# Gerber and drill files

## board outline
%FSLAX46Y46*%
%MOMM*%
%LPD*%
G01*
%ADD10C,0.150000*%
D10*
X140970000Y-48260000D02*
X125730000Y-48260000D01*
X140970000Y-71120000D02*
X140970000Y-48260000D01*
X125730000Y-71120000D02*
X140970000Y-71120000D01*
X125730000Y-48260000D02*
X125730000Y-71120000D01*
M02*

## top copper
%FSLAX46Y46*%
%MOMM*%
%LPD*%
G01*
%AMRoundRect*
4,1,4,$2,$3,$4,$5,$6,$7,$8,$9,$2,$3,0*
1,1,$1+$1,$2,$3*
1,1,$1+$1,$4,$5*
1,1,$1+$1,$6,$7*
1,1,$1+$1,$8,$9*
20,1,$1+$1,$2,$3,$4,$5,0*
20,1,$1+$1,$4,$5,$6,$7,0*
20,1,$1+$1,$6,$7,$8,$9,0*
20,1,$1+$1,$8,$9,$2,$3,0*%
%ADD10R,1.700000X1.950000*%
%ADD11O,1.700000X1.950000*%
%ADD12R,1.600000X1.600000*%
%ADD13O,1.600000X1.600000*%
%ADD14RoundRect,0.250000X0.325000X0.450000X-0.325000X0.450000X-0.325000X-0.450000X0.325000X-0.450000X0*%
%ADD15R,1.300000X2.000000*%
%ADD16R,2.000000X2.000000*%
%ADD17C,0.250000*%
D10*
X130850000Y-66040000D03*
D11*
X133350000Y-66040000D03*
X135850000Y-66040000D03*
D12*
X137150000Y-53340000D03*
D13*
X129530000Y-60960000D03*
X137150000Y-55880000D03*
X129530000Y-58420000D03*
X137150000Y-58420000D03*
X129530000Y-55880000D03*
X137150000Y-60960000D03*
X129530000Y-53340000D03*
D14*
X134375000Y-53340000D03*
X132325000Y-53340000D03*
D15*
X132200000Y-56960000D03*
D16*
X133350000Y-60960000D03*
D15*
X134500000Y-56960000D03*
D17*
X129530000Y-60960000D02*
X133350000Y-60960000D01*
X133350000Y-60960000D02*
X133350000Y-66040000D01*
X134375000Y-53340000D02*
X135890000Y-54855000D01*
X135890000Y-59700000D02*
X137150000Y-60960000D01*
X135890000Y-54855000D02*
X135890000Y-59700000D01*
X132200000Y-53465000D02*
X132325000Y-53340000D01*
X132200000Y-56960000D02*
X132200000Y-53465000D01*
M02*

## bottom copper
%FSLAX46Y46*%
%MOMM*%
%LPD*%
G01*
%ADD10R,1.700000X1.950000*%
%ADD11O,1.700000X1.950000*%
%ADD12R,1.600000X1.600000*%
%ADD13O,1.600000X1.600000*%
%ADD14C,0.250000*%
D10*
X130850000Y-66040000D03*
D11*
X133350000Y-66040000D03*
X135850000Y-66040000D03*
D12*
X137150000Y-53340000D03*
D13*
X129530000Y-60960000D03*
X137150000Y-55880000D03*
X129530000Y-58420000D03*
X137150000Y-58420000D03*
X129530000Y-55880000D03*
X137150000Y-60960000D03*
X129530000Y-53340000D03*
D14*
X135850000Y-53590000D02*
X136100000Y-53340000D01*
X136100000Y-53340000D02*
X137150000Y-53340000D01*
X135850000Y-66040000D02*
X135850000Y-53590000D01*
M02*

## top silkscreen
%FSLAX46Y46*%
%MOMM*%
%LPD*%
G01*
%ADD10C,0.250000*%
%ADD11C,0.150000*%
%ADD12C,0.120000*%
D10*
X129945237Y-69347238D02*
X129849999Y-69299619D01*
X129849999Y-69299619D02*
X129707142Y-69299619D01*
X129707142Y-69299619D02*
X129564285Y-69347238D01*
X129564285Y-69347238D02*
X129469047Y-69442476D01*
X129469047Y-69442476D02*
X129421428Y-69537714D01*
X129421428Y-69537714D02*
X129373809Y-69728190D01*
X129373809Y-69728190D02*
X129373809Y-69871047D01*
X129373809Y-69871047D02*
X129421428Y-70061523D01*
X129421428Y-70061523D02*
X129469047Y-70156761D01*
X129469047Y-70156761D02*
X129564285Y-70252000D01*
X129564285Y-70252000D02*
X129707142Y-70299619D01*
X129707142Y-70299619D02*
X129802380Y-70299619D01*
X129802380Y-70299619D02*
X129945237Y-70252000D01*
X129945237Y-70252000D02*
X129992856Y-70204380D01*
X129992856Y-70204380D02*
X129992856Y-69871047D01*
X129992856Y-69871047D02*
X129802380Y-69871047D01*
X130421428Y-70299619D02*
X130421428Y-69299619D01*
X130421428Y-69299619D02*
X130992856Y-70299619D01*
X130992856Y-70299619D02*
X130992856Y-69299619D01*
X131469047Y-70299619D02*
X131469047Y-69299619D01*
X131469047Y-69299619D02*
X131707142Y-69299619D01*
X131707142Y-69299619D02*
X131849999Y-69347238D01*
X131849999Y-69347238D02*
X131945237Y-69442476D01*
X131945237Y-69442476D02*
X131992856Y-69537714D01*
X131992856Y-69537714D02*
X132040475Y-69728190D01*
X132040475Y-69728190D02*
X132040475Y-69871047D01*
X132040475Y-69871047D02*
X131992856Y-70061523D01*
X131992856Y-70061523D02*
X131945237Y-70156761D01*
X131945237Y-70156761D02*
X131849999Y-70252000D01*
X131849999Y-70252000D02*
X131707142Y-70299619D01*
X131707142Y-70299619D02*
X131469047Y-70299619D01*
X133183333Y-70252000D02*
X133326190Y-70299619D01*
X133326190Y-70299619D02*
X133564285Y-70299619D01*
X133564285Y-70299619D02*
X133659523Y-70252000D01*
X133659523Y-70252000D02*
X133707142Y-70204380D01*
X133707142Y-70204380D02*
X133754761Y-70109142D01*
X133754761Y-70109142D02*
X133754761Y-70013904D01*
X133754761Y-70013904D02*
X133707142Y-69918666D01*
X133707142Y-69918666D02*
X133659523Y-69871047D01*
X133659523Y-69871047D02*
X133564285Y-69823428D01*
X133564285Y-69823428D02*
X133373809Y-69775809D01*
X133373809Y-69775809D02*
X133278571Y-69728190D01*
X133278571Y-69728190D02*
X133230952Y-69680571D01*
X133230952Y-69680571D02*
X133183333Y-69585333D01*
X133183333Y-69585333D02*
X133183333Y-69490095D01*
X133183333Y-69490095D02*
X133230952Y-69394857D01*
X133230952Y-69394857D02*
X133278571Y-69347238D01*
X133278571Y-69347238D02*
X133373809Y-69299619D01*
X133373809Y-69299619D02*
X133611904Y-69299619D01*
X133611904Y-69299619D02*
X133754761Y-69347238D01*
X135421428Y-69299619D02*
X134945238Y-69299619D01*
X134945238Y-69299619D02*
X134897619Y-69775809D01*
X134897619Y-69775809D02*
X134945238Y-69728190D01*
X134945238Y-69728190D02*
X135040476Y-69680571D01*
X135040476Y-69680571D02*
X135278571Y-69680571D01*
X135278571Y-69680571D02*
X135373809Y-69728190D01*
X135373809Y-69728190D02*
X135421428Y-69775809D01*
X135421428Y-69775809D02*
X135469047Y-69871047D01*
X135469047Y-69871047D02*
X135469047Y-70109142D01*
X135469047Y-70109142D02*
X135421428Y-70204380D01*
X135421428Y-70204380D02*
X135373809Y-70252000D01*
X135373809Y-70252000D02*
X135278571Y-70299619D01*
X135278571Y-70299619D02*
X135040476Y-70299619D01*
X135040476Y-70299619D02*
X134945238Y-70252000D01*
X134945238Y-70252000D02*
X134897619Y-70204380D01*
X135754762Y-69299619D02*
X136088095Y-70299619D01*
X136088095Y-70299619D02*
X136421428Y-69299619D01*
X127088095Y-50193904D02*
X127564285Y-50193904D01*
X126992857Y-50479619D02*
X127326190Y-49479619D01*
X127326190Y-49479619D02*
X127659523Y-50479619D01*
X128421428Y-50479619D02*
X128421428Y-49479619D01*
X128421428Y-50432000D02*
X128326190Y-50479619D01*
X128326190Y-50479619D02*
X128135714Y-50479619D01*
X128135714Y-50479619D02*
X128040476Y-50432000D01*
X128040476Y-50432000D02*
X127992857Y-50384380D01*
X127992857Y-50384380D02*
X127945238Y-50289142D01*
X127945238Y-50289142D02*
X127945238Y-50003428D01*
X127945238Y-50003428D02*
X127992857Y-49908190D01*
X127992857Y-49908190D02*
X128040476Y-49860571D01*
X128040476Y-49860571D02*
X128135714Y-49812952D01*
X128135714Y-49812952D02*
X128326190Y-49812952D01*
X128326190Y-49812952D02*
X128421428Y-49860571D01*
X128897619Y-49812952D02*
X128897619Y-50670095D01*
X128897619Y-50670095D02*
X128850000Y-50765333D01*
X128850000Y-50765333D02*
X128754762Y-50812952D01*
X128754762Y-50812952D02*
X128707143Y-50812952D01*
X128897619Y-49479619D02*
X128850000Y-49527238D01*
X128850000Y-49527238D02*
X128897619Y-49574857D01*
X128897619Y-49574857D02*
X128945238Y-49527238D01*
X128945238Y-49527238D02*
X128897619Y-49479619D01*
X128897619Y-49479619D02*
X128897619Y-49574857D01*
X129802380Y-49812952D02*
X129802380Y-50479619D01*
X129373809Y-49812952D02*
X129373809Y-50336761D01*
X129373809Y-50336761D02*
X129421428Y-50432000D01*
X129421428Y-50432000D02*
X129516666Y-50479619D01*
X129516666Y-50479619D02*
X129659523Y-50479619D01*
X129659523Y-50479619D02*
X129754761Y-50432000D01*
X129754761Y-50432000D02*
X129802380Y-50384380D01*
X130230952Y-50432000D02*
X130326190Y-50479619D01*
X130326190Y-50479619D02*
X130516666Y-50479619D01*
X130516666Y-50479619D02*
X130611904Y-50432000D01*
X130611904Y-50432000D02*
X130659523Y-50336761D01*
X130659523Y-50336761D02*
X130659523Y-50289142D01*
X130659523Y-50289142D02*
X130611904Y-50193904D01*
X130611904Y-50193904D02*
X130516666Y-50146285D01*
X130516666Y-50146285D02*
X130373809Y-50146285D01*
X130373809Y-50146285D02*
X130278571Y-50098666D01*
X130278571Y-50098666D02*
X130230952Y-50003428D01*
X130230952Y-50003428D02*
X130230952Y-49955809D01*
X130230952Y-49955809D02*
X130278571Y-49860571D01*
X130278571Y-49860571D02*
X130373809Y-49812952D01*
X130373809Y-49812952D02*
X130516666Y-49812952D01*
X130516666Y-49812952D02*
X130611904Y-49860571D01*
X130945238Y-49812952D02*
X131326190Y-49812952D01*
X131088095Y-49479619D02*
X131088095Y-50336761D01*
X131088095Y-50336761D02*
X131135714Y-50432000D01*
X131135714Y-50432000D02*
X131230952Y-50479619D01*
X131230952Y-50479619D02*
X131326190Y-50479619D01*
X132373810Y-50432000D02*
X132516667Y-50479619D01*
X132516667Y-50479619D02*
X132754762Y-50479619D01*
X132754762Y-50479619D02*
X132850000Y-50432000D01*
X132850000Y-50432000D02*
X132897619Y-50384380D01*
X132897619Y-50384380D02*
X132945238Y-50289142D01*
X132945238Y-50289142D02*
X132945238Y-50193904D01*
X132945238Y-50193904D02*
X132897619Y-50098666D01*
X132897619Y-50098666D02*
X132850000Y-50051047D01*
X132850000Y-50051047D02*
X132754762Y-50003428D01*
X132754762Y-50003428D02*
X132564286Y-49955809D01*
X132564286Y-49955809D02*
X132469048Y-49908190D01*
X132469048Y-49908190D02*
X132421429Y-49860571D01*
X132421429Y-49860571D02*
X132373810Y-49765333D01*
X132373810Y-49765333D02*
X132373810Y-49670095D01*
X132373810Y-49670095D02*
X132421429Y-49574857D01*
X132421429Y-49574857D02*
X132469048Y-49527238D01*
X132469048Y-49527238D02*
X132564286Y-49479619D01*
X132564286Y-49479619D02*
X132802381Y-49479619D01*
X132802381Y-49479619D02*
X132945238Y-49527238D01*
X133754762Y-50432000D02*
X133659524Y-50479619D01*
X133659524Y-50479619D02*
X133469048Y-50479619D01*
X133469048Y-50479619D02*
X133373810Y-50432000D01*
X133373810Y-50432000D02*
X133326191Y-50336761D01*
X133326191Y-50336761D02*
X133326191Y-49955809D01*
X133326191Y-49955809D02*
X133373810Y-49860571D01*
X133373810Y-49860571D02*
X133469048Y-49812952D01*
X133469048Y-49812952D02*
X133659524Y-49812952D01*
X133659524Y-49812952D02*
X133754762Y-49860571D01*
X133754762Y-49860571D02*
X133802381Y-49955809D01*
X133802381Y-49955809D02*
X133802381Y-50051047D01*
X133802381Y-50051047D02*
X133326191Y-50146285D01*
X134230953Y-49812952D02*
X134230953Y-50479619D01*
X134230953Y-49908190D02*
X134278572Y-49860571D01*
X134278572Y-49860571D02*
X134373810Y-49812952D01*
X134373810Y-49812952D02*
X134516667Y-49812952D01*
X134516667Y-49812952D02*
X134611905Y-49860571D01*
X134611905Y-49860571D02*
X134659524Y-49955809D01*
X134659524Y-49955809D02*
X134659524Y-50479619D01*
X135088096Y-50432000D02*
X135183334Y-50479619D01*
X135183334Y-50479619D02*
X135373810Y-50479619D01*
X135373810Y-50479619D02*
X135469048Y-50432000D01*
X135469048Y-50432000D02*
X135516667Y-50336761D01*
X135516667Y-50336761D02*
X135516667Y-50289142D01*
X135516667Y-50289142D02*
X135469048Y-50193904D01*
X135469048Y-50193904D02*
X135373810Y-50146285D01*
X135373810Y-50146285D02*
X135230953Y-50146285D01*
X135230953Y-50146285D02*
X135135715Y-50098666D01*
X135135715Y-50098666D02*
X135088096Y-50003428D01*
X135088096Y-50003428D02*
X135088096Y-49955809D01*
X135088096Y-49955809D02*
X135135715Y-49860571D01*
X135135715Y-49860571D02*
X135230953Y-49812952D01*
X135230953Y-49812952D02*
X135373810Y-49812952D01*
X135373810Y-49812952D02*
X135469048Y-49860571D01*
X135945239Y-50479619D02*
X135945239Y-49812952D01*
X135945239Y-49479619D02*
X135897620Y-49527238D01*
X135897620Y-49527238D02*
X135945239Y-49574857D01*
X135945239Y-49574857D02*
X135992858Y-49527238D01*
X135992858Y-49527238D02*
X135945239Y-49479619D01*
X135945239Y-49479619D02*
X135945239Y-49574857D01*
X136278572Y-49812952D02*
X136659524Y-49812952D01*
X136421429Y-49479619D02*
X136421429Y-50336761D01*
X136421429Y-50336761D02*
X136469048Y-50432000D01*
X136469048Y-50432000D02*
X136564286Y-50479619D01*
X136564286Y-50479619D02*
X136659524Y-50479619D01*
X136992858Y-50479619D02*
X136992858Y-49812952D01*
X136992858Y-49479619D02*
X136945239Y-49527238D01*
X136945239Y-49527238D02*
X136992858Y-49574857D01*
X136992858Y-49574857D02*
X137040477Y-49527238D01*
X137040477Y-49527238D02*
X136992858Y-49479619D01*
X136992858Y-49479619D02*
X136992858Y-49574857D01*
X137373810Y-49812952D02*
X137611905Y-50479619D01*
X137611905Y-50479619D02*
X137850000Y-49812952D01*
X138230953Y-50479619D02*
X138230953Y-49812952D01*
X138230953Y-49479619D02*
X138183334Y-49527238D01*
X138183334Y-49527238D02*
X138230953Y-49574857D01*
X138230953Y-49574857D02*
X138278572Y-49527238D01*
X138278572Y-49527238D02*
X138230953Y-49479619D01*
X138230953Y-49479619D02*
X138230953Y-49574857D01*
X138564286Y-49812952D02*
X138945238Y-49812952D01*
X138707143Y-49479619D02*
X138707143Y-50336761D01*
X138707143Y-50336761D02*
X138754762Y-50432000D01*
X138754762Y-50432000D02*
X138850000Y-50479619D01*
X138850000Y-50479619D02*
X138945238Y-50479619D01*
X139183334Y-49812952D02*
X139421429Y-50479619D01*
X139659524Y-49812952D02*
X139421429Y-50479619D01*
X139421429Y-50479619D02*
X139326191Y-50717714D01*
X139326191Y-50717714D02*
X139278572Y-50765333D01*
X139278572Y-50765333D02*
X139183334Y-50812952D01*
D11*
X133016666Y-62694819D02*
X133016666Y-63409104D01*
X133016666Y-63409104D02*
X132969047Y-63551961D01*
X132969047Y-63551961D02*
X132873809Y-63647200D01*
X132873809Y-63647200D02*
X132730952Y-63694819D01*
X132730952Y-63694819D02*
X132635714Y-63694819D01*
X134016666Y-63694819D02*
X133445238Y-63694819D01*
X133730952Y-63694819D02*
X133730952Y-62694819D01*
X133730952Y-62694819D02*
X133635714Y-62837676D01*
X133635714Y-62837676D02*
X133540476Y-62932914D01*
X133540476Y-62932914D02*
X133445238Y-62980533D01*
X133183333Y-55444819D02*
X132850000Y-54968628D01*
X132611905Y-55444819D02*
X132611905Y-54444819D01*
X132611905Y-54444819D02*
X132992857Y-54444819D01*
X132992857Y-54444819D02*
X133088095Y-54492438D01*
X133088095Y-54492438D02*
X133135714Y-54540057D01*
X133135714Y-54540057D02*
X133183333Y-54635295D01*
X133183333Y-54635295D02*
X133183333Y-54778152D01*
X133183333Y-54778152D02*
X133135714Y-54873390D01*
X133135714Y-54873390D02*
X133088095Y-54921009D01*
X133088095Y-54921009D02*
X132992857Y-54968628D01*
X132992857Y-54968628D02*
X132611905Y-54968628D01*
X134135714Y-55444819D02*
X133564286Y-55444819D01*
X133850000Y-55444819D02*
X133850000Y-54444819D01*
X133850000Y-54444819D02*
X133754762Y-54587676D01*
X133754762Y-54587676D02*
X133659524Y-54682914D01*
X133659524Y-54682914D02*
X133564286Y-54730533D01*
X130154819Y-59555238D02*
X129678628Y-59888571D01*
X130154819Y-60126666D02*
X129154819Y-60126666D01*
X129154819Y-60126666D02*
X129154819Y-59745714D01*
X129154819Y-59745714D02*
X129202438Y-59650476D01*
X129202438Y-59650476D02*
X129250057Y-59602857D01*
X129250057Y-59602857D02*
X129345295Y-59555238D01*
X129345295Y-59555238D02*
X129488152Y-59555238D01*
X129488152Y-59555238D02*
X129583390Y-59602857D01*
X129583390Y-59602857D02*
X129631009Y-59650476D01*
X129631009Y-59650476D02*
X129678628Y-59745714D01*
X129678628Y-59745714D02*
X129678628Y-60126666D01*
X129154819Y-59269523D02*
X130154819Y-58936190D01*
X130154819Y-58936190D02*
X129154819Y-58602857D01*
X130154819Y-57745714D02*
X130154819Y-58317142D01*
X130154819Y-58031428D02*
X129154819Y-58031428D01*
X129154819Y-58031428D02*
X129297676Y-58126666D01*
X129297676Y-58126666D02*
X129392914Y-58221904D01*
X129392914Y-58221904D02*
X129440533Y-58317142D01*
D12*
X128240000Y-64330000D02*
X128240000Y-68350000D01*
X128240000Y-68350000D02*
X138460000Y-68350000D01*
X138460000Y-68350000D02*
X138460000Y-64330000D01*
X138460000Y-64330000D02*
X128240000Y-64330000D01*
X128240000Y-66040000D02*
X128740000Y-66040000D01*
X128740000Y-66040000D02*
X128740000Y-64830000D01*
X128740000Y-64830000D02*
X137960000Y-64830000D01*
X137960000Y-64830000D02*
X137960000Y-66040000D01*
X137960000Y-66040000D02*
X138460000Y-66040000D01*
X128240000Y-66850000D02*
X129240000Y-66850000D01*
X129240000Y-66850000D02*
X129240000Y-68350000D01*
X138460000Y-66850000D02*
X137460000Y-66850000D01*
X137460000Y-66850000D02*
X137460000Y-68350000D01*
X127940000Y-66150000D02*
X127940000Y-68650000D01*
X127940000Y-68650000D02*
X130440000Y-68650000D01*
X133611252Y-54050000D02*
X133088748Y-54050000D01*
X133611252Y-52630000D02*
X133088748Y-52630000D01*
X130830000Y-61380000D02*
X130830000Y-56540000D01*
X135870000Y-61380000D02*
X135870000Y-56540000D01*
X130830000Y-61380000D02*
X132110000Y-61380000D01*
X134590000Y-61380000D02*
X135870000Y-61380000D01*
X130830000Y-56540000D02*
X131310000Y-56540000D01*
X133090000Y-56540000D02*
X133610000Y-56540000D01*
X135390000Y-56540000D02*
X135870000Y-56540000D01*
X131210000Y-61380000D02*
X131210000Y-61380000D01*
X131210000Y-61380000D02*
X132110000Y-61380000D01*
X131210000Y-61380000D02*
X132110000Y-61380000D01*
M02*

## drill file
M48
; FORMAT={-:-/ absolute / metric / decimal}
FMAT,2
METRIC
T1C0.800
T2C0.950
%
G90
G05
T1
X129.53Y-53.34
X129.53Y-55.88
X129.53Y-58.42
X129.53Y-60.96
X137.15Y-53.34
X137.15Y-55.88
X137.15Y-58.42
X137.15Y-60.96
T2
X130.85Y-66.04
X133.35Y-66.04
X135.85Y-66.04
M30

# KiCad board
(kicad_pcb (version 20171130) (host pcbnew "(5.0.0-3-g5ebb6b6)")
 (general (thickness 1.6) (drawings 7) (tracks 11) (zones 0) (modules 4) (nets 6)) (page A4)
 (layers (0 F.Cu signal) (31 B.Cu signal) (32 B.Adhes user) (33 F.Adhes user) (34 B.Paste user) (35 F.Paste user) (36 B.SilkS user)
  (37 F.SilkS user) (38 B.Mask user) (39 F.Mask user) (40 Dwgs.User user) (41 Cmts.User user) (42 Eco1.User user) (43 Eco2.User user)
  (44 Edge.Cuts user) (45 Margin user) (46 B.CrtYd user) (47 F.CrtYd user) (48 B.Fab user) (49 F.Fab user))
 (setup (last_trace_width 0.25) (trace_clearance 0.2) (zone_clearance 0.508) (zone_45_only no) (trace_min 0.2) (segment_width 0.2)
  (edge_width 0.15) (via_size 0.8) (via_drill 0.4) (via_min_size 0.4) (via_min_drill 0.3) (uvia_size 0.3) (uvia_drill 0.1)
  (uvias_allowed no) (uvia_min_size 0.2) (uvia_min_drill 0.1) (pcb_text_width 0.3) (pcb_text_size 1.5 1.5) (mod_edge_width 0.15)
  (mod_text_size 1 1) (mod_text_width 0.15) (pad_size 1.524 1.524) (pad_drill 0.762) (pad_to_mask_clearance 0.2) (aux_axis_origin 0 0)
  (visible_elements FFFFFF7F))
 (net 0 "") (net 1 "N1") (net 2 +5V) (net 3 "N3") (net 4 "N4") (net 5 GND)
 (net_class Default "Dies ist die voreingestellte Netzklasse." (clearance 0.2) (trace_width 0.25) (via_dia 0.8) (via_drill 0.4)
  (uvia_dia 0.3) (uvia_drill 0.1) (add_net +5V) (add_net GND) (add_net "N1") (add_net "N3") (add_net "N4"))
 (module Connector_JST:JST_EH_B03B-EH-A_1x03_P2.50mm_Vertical (layer F.Cu) (at 130.85 66.04)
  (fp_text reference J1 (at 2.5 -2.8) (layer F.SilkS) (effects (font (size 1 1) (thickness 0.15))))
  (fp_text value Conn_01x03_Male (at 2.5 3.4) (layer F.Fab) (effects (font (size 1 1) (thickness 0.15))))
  (fp_line (start -2.61 -1.71) (end -2.61 2.31) (layer F.SilkS) (width 0.12))
  (fp_line (start -2.61 2.31) (end 7.61 2.31) (layer F.SilkS) (width 0.12))
  (fp_line (start 7.61 2.31) (end 7.61 -1.71) (layer F.SilkS) (width 0.12))
  (fp_line (start 7.61 -1.71) (end -2.61 -1.71) (layer F.SilkS) (width 0.12))
  (fp_line (start -2.61 0) (end -2.11 0) (layer F.SilkS) (width 0.12))
  (fp_line (start -2.11 0) (end -2.11 -1.21) (layer F.SilkS) (width 0.12))
  (fp_line (start -2.11 -1.21) (end 7.11 -1.21) (layer F.SilkS) (width 0.12))
  (fp_line (start 7.11 -1.21) (end 7.11 0) (layer F.SilkS) (width 0.12))
  (fp_line (start 7.11 0) (end 7.61 0) (layer F.SilkS) (width 0.12))
  (fp_line (start -2.61 0.81) (end -1.61 0.81) (layer F.SilkS) (width 0.12))
  (fp_line (start -1.61 0.81) (end -1.61 2.31) (layer F.SilkS) (width 0.12))
  (fp_line (start 7.61 0.81) (end 6.61 0.81) (layer F.SilkS) (width 0.12))
  (fp_line (start 6.61 0.81) (end 6.61 2.31) (layer F.SilkS) (width 0.12))
  (fp_line (start -2.91 0.11) (end -2.91 2.61) (layer F.SilkS) (width 0.12))
  (fp_line (start -2.91 2.61) (end -0.41 2.61) (layer F.SilkS) (width 0.12))
  (pad 1 thru_hole rect (at 0 0) (size 1.7 1.95) (drill 0.95) (layers *.Cu *.Mask))
  (pad 2 thru_hole oval (at 2.5 0) (size 1.7 1.95) (drill 0.95) (layers *.Cu *.Mask) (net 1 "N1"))
  (pad 3 thru_hole oval (at 5 0) (size 1.7 1.95) (drill 0.95) (layers *.Cu *.Mask) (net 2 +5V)))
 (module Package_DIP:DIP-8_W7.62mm (layer B.Cu) (at 137.15 53.34 180)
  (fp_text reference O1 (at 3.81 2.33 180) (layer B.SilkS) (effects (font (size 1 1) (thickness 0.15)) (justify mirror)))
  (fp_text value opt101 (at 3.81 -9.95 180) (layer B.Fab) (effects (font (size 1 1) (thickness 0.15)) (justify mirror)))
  (pad 1 thru_hole rect (at 0 0 180) (size 1.6 1.6) (drill 0.8) (layers *.Cu *.Mask) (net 2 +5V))
  (pad 5 thru_hole oval (at 7.62 -7.62 180) (size 1.6 1.6) (drill 0.8) (layers *.Cu *.Mask) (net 1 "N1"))
  (pad 2 thru_hole oval (at 0 -2.54 180) (size 1.6 1.6) (drill 0.8) (layers *.Cu *.Mask))
  (pad 6 thru_hole oval (at 7.62 -5.08 180) (size 1.6 1.6) (drill 0.8) (layers *.Cu *.Mask))
  (pad 3 thru_hole oval (at 0 -5.08 180) (size 1.6 1.6) (drill 0.8) (layers *.Cu *.Mask))
  (pad 7 thru_hole oval (at 7.62 -2.54 180) (size 1.6 1.6) (drill 0.8) (layers *.Cu *.Mask))
  (pad 4 thru_hole oval (at 0 -7.62 180) (size 1.6 1.6) (drill 0.8) (layers *.Cu *.Mask) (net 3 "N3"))
  (pad 8 thru_hole oval (at 7.62 0 180) (size 1.6 1.6) (drill 0.8) (layers *.Cu *.Mask)))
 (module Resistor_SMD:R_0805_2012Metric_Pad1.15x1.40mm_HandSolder (layer F.Cu) (at 133.35 53.34 180)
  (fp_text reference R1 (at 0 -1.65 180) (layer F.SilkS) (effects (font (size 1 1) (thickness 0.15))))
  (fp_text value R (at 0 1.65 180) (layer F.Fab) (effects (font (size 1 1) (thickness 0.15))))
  (fp_line (start -0.261252 -0.71) (end 0.261252 -0.71) (layer F.SilkS) (width 0.12))
  (fp_line (start -0.261252 0.71) (end 0.261252 0.71) (layer F.SilkS) (width 0.12))
  (pad 1 smd roundrect (at -1.025 0 180) (size 1.15 1.4) (layers F.Cu F.Paste F.Mask) (roundrect_rratio 0.217391) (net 3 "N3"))
  (pad 2 smd roundrect (at 1.025 0 180) (size 1.15 1.4) (layers F.Cu F.Paste F.Mask) (roundrect_rratio 0.217391) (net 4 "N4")))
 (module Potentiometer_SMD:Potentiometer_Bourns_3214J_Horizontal (layer F.Cu) (at 133.35 58.96 90)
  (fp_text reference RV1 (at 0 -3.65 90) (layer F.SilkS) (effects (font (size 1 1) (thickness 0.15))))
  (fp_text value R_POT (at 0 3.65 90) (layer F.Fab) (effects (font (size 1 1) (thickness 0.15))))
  (fp_line (start -2.42 -2.52) (end 2.42 -2.52) (layer F.SilkS) (width 0.12))
  (fp_line (start -2.42 2.52) (end 2.42 2.52) (layer F.SilkS) (width 0.12))
  (fp_line (start -2.42 -2.52) (end -2.42 -1.24) (layer F.SilkS) (width 0.12))
  (fp_line (start -2.42 1.24) (end -2.42 2.52) (layer F.SilkS) (width 0.12))
  (fp_line (start 2.42 -2.52) (end 2.42 -2.04) (layer F.SilkS) (width 0.12))
  (fp_line (start 2.42 -0.26) (end 2.42 0.26) (layer F.SilkS) (width 0.12))
  (fp_line (start 2.42 2.04) (end 2.42 2.52) (layer F.SilkS) (width 0.12))
  (fp_line (start -2.42 -2.14) (end -2.42 -2.14) (layer F.SilkS) (width 0.12))
  (fp_line (start -2.42 -2.14) (end -2.42 -1.24) (layer F.SilkS) (width 0.12))
  (fp_line (start -2.42 -2.14) (end -2.42 -1.24) (layer F.SilkS) (width 0.12))
  (pad 1 smd rect (at 2 -1.15 90) (size 2 1.3) (layers F.Cu F.Paste F.Mask) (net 4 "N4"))
  (pad 2 smd rect (at -2 0 90) (size 2 2) (layers F.Cu F.Paste F.Mask) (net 1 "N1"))
  (pad 3 smd rect (at 2 1.15 90) (size 2 1.3) (layers F.Cu F.Paste F.Mask)))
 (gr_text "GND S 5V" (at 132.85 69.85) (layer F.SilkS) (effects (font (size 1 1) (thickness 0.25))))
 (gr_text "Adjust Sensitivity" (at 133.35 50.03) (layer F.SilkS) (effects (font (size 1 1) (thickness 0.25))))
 (gr_line (start 140.97 48.26) (end 125.73 48.26) (layer Edge.Cuts) (width 0.15))
 (gr_line (start 140.97 71.12) (end 140.97 48.26) (layer Edge.Cuts) (width 0.15))
 (gr_line (start 125.73 71.12) (end 140.97 71.12) (layer Edge.Cuts) (width 0.15))
 (gr_line (start 125.73 48.26) (end 125.73 71.12) (layer Edge.Cuts) (width 0.15))
 (segment (start 129.53 60.96) (end 133.35 60.96) (width 0.25) (layer F.Cu) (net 1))
 (segment (start 133.35 60.96) (end 133.35 66.04) (width 0.25) (layer F.Cu) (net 1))
 (segment (start 135.85 53.59) (end 136.1 53.34) (width 0.25) (layer B.Cu) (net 2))
 (segment (start 136.1 53.34) (end 137.15 53.34) (width 0.25) (layer B.Cu) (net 2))
 (segment (start 135.85 66.04) (end 135.85 53.59) (width 0.25) (layer B.Cu) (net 2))
 (segment (start 134.375 53.34) (end 135.89 54.855) (width 0.25) (layer F.Cu) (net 3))
 (segment (start 135.89 59.7) (end 137.15 60.96) (width 0.25) (layer F.Cu) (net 3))
 (segment (start 135.89 54.855) (end 135.89 59.7) (width 0.25) (layer F.Cu) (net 3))
 (segment (start 132.2 53.465) (end 132.325 53.34) (width 0.25) (layer F.Cu) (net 4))
 (segment (start 132.2 56.96) (end 132.2 53.465) (width 0.25) (layer F.Cu) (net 4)))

